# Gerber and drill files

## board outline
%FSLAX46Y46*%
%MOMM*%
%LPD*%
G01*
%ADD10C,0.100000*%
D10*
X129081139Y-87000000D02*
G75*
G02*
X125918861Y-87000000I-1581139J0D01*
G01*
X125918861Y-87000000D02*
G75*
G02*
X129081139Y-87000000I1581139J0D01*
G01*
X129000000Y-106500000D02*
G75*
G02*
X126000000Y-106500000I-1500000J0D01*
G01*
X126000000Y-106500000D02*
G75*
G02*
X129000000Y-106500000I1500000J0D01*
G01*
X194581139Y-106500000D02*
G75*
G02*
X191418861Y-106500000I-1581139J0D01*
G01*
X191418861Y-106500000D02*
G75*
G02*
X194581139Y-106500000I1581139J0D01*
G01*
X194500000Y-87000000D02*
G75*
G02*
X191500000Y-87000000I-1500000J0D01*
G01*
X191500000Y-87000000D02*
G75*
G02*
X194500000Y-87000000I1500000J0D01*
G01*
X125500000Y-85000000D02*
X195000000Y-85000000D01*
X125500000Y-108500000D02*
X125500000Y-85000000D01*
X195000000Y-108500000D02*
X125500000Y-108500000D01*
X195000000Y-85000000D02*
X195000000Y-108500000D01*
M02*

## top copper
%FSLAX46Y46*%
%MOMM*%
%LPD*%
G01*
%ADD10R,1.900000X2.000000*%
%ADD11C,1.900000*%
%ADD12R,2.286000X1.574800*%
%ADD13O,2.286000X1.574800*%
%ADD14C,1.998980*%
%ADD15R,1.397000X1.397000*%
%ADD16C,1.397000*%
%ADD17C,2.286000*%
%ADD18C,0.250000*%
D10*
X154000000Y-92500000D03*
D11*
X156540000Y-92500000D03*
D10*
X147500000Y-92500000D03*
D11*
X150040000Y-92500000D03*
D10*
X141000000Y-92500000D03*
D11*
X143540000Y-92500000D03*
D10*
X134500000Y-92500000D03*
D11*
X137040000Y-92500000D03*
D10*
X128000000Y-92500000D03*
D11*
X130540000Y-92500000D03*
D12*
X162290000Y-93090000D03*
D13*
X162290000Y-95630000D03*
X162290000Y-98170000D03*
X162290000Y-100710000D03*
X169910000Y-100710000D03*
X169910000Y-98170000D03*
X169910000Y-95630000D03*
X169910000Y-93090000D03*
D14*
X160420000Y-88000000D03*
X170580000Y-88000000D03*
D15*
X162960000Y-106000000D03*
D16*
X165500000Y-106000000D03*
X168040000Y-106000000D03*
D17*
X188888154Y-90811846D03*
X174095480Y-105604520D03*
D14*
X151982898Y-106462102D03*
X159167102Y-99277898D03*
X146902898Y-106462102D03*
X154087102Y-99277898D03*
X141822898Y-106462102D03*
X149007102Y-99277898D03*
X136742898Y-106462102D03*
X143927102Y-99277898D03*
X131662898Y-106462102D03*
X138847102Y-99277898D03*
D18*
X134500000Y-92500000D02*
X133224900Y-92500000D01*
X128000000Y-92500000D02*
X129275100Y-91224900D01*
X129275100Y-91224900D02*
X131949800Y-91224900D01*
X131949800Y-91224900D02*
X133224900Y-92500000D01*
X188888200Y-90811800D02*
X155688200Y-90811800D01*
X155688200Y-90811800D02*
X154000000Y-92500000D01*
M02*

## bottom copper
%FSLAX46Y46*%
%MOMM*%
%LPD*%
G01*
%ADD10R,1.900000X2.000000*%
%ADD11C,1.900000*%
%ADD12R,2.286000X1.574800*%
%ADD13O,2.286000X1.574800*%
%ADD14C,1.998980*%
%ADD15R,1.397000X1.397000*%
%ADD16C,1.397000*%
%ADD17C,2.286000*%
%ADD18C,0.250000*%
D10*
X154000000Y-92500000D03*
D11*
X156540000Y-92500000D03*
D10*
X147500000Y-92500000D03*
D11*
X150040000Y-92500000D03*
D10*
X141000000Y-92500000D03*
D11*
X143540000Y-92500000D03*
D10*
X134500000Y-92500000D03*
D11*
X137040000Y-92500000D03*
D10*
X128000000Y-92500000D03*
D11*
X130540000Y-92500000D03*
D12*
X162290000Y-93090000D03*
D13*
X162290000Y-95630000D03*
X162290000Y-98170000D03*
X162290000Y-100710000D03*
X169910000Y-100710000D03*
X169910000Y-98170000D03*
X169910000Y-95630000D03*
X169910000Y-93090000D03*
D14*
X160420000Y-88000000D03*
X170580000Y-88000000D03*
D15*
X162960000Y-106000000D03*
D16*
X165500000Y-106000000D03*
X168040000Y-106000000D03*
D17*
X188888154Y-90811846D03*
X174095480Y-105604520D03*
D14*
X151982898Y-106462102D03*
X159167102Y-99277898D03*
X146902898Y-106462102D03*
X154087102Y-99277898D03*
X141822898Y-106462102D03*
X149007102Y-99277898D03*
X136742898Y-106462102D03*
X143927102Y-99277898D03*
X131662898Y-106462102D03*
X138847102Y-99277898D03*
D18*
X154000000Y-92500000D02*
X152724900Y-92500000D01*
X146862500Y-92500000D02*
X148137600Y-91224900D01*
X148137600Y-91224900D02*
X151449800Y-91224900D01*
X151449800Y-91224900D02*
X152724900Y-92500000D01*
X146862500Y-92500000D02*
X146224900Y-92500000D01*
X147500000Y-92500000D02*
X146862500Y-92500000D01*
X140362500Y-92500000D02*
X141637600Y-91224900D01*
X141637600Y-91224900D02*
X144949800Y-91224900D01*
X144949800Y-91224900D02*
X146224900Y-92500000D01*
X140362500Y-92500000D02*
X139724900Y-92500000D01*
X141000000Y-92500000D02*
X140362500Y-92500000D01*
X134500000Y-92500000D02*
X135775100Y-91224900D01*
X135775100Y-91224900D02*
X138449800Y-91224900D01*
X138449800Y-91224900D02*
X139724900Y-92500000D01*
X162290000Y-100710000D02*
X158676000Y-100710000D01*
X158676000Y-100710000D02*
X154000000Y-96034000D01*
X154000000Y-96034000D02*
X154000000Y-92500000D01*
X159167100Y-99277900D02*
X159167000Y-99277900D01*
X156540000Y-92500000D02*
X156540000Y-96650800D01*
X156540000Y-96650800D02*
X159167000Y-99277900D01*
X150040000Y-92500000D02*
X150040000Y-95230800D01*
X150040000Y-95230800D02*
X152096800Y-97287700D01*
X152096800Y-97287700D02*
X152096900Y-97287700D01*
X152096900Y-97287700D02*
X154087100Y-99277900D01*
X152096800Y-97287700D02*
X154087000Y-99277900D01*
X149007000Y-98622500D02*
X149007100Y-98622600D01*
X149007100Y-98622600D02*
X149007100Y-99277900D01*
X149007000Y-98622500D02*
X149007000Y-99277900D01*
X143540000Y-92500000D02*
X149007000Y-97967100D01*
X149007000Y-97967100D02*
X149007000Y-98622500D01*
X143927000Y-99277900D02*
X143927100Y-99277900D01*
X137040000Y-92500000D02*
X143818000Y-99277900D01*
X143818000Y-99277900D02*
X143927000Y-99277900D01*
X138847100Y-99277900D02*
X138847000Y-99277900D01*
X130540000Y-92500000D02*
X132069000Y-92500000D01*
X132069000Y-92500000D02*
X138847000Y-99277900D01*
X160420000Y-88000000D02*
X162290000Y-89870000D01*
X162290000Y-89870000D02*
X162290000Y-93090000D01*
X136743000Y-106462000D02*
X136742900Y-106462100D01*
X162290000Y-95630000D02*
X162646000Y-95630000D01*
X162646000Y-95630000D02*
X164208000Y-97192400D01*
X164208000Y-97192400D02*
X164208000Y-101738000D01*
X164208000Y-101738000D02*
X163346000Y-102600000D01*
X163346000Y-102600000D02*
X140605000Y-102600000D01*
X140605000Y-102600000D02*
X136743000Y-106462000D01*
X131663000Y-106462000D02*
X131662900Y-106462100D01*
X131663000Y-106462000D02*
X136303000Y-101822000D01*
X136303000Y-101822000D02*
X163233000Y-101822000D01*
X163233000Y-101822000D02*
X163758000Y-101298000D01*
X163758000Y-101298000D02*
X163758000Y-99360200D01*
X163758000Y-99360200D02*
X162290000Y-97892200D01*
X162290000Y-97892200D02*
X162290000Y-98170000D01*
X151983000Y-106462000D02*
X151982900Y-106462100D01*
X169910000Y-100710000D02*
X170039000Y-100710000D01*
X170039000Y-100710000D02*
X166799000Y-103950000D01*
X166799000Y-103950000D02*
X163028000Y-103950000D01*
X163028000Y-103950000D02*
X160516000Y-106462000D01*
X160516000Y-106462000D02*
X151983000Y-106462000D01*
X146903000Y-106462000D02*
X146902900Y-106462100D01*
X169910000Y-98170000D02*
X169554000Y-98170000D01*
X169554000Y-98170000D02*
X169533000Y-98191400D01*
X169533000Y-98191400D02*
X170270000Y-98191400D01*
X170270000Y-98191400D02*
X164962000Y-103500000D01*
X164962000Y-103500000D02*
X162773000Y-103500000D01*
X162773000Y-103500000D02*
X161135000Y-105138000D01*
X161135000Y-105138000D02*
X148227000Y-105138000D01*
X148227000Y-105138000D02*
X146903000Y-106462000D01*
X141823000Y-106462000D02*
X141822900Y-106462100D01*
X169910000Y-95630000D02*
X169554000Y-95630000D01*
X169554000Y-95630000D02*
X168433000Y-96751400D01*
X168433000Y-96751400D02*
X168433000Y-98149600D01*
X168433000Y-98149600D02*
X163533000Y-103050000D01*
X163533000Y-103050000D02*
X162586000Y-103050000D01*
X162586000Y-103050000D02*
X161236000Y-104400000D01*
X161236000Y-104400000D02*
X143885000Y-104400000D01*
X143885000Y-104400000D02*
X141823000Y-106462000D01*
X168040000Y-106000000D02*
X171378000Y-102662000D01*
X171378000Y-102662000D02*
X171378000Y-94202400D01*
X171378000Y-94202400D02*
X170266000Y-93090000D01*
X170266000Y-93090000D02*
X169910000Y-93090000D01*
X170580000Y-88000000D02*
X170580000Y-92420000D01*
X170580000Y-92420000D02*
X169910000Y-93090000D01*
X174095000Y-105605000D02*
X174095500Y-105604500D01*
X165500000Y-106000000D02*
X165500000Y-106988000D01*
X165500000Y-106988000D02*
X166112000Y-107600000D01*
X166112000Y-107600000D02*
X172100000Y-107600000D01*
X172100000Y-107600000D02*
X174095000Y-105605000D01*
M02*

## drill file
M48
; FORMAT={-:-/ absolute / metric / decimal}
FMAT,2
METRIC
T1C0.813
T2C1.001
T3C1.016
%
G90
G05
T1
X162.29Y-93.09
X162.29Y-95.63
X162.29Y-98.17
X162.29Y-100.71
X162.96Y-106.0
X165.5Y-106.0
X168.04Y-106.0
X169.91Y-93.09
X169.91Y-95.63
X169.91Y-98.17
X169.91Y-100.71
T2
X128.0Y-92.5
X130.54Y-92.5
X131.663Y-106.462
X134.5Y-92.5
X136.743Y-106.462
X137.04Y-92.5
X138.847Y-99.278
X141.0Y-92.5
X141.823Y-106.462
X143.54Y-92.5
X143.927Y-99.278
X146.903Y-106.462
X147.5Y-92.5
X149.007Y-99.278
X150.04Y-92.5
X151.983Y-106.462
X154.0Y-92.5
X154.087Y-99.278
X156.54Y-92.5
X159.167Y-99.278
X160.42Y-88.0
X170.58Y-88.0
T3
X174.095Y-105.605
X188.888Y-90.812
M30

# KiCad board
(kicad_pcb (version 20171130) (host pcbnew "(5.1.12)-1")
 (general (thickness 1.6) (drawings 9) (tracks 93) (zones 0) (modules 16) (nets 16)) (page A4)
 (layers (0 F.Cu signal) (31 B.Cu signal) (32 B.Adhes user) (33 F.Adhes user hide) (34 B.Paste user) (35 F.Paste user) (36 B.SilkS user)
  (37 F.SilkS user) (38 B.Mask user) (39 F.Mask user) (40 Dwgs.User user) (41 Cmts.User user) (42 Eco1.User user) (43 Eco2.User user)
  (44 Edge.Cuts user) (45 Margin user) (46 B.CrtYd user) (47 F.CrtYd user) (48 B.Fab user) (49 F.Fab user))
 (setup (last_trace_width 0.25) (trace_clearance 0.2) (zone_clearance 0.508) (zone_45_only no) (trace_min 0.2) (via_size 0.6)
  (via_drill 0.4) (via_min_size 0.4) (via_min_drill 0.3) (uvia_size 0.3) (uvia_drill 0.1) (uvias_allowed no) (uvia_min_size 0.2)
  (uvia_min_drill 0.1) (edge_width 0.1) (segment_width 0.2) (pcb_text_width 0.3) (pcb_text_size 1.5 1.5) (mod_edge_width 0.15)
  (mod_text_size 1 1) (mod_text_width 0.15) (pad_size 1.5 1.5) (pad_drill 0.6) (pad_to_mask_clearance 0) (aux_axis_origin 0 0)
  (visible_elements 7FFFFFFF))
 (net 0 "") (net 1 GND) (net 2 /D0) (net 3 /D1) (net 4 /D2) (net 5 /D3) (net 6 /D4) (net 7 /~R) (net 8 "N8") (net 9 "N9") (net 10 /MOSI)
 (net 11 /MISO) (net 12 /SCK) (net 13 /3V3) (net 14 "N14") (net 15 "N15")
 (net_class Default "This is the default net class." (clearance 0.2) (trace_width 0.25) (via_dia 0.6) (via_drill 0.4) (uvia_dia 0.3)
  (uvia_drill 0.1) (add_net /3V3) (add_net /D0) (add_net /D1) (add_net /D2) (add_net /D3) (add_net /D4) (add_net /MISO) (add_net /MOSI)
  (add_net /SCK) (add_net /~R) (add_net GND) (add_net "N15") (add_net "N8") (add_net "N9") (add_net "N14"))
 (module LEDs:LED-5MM (layer F.Cu) (at 154 92.5)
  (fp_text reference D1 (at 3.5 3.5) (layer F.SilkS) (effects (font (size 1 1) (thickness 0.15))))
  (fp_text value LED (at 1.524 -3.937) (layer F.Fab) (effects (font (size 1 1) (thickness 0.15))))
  (pad 1 thru_hole rect (at 0 0 90) (size 2 1.9) (drill 1.00076) (layers *.Cu *.Mask F.SilkS) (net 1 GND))
  (pad 2 thru_hole circle (at 2.54 0) (size 1.9 1.9) (drill 1.00076) (layers *.Cu *.Mask F.SilkS) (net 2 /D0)))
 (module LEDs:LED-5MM (layer F.Cu) (at 147.5 92.5)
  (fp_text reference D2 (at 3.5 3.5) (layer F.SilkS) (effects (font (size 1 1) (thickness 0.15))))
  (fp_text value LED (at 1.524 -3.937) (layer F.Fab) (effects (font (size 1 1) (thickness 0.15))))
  (pad 1 thru_hole rect (at 0 0 90) (size 2 1.9) (drill 1.00076) (layers *.Cu *.Mask F.SilkS) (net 1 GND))
  (pad 2 thru_hole circle (at 2.54 0) (size 1.9 1.9) (drill 1.00076) (layers *.Cu *.Mask F.SilkS) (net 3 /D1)))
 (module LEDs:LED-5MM (layer F.Cu) (at 141 92.5)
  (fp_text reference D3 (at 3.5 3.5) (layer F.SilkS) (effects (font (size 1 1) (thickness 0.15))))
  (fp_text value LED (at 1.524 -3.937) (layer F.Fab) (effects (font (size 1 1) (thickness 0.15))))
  (pad 1 thru_hole rect (at 0 0 90) (size 2 1.9) (drill 1.00076) (layers *.Cu *.Mask F.SilkS) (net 1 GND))
  (pad 2 thru_hole circle (at 2.54 0) (size 1.9 1.9) (drill 1.00076) (layers *.Cu *.Mask F.SilkS) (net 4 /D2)))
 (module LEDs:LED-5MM (layer F.Cu) (at 134.5 92.5)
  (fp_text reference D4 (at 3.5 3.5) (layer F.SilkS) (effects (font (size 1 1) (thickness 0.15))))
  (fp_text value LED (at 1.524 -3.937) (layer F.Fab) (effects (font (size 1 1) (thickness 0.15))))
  (pad 1 thru_hole rect (at 0 0 90) (size 2 1.9) (drill 1.00076) (layers *.Cu *.Mask F.SilkS) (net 1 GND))
  (pad 2 thru_hole circle (at 2.54 0) (size 1.9 1.9) (drill 1.00076) (layers *.Cu *.Mask F.SilkS) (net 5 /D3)))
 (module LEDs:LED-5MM (layer F.Cu) (at 128 92.5)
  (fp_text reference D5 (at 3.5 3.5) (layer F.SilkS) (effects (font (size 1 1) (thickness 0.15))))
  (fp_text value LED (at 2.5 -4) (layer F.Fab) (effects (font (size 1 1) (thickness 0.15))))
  (pad 1 thru_hole rect (at 0 0 90) (size 2 1.9) (drill 1.00076) (layers *.Cu *.Mask F.SilkS) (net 1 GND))
  (pad 2 thru_hole circle (at 2.54 0) (size 1.9 1.9) (drill 1.00076) (layers *.Cu *.Mask F.SilkS) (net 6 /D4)))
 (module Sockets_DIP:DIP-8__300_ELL (layer F.Cu) (at 166.1 96.9 270)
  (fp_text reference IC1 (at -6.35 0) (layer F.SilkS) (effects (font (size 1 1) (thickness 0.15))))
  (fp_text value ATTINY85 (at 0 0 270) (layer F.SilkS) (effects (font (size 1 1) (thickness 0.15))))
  (pad 1 thru_hole rect (at -3.81 3.81 270) (size 1.5748 2.286) (drill 0.8128) (layers *.Cu *.Mask F.SilkS) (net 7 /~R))
  (pad 2 thru_hole oval (at -1.27 3.81 270) (size 1.5748 2.286) (drill 0.8128) (layers *.Cu *.Mask F.SilkS) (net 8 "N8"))
  (pad 3 thru_hole oval (at 1.27 3.81 270) (size 1.5748 2.286) (drill 0.8128) (layers *.Cu *.Mask F.SilkS) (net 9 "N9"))
  (pad 4 thru_hole oval (at 3.81 3.81 270) (size 1.5748 2.286) (drill 0.8128) (layers *.Cu *.Mask F.SilkS) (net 1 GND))
  (pad 5 thru_hole oval (at 3.81 -3.81 270) (size 1.5748 2.286) (drill 0.8128) (layers *.Cu *.Mask F.SilkS) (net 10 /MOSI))
  (pad 6 thru_hole oval (at 1.27 -3.81 270) (size 1.5748 2.286) (drill 0.8128) (layers *.Cu *.Mask F.SilkS) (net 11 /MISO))
  (pad 7 thru_hole oval (at -1.27 -3.81 270) (size 1.5748 2.286) (drill 0.8128) (layers *.Cu *.Mask F.SilkS) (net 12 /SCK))
  (pad 8 thru_hole oval (at -3.81 -3.81 270) (size 1.5748 2.286) (drill 0.8128) (layers *.Cu *.Mask F.SilkS) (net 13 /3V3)))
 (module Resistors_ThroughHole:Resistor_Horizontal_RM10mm (layer F.Cu) (at 165.5 88)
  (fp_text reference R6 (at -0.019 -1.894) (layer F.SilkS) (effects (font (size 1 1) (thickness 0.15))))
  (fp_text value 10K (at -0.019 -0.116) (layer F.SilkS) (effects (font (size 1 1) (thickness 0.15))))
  (pad 1 thru_hole circle (at -5.08 0) (size 1.99898 1.99898) (drill 1.00076) (layers *.Cu *.SilkS *.Mask) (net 7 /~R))
  (pad 2 thru_hole circle (at 5.08 0) (size 1.99898 1.99898) (drill 1.00076) (layers *.Cu *.SilkS *.Mask) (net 13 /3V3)))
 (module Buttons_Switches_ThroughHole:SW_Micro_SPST (layer F.Cu) (at 165.5 106)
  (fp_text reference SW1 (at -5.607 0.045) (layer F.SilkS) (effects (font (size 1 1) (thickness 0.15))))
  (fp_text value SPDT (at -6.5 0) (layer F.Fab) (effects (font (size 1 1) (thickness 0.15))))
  (pad 1 thru_hole rect (at -2.54 0) (size 1.397 1.397) (drill 0.8128) (layers *.Cu *.Mask F.SilkS) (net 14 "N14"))
  (pad 2 thru_hole circle (at 0 0) (size 1.397 1.397) (drill 0.8128) (layers *.Cu *.Mask F.SilkS) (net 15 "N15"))
  (pad 3 thru_hole circle (at 2.54 0) (size 1.397 1.397) (drill 0.8128) (layers *.Cu *.Mask F.SilkS) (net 13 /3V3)))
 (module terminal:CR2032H (layer F.Cu) (at 183.5 96.2 225)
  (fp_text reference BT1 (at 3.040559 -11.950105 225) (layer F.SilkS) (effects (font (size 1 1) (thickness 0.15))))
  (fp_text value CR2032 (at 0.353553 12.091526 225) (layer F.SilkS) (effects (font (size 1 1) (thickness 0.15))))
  (pad 2 thru_hole circle (at -7.62 0 225) (size 2.286 2.286) (drill 1.016) (layers *.Cu *.Mask F.SilkS) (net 1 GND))
  (pad 1 thru_hole circle (at 13.3 0 225) (size 2.286 2.286) (drill 1.016) (layers *.Cu *.Mask F.SilkS) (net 15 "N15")))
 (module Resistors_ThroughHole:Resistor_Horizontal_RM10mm (layer F.Cu) (at 155.575 102.87 45)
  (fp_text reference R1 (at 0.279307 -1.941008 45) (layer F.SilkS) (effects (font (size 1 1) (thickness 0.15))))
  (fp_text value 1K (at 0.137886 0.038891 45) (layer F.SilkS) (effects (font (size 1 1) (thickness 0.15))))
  (pad 1 thru_hole circle (at -5.08 0 45) (size 1.99898 1.99898) (drill 1.00076) (layers *.Cu *.SilkS *.Mask) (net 10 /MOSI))
  (pad 2 thru_hole circle (at 5.08 0 45) (size 1.99898 1.99898) (drill 1.00076) (layers *.Cu *.SilkS *.Mask) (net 2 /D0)))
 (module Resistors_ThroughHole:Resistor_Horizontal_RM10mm (layer F.Cu) (at 150.495 102.87 45)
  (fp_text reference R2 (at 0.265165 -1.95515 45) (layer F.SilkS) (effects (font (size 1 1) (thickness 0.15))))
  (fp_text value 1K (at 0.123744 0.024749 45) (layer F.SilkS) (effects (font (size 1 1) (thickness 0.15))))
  (pad 1 thru_hole circle (at -5.08 0 45) (size 1.99898 1.99898) (drill 1.00076) (layers *.Cu *.SilkS *.Mask) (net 11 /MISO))
  (pad 2 thru_hole circle (at 5.08 0 45) (size 1.99898 1.99898) (drill 1.00076) (layers *.Cu *.SilkS *.Mask) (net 3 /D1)))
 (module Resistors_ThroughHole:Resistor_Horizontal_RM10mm (layer F.Cu) (at 145.415 102.87 45)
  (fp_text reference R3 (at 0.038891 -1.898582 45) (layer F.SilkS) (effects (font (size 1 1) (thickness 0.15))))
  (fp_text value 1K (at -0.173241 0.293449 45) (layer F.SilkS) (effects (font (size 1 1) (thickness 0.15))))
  (pad 1 thru_hole circle (at -5.08 0 45) (size 1.99898 1.99898) (drill 1.00076) (layers *.Cu *.SilkS *.Mask) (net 12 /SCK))
  (pad 2 thru_hole circle (at 5.08 0 45) (size 1.99898 1.99898) (drill 1.00076) (layers *.Cu *.SilkS *.Mask) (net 4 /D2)))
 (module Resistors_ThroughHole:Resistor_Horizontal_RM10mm (layer F.Cu) (at 140.335 102.87 45)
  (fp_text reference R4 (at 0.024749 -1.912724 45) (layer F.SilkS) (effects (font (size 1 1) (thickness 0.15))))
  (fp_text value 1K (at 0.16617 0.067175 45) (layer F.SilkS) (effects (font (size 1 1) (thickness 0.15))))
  (pad 1 thru_hole circle (at -5.08 0 45) (size 1.99898 1.99898) (drill 1.00076) (layers *.Cu *.SilkS *.Mask) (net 8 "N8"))
  (pad 2 thru_hole circle (at 5.08 0 45) (size 1.99898 1.99898) (drill 1.00076) (layers *.Cu *.SilkS *.Mask) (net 5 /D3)))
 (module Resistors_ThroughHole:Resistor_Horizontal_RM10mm (layer F.Cu) (at 135.255 102.87 45)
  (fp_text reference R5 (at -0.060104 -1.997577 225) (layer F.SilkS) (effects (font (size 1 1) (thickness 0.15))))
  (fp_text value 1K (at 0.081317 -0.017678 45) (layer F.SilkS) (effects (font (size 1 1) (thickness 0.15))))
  (pad 1 thru_hole circle (at -5.08 0 45) (size 1.99898 1.99898) (drill 1.00076) (layers *.Cu *.SilkS *.Mask) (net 9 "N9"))
  (pad 2 thru_hole circle (at 5.08 0 45) (size 1.99898 1.99898) (drill 1.00076) (layers *.Cu *.SilkS *.Mask) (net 6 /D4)))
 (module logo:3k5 (layer F.Cu) (at 140.589 87.503)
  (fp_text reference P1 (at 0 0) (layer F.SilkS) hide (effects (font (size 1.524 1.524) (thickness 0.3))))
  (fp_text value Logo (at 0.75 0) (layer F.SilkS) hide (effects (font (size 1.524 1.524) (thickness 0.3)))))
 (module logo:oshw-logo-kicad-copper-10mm (layer F.Cu) (at 129.413 99.187)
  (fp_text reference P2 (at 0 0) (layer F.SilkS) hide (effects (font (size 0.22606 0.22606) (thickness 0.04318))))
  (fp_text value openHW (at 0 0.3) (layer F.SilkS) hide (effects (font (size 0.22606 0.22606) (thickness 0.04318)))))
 (gr_circle (center 127.5 87) (end 129 87.5) (layer Edge.Cuts) (width 0.1))
 (gr_circle (center 127.5 106.5) (end 129 106.5) (layer Edge.Cuts) (width 0.1))
 (gr_circle (center 193 106.5) (end 194.5 107) (layer Edge.Cuts) (width 0.1))
 (gr_circle (center 193 87) (end 194.5 87) (layer Edge.Cuts) (width 0.1))
 (gr_line (start 125.5 85) (end 195 85) (angle 90) (layer Edge.Cuts) (width 0.1))
 (gr_line (start 125.5 108.5) (end 125.5 85) (angle 90) (layer Edge.Cuts) (width 0.1))
 (gr_line (start 195 108.5) (end 125.5 108.5) (angle 90) (layer Edge.Cuts) (width 0.1))
 (gr_line (start 195 85) (end 195 108.5) (angle 90) (layer Edge.Cuts) (width 0.1))
 (segment (start 154 92.5) (end 152.7249 92.5) (width 0.25) (layer B.Cu) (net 1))
 (segment (start 146.8625 92.5) (end 148.1376 91.2249) (width 0.25) (layer B.Cu) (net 1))
 (segment (start 148.1376 91.2249) (end 151.4498 91.2249) (width 0.25) (layer B.Cu) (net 1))
 (segment (start 151.4498 91.2249) (end 152.7249 92.5) (width 0.25) (layer B.Cu) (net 1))
 (segment (start 146.8625 92.5) (end 146.2249 92.5) (width 0.25) (layer B.Cu) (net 1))
 (segment (start 147.5 92.5) (end 146.8625 92.5) (width 0.25) (layer B.Cu) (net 1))
 (segment (start 140.3625 92.5) (end 141.6376 91.2249) (width 0.25) (layer B.Cu) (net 1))
 (segment (start 141.6376 91.2249) (end 144.9498 91.2249) (width 0.25) (layer B.Cu) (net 1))
 (segment (start 144.9498 91.2249) (end 146.2249 92.5) (width 0.25) (layer B.Cu) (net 1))
 (segment (start 140.3625 92.5) (end 139.7249 92.5) (width 0.25) (layer B.Cu) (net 1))
 (segment (start 141 92.5) (end 140.3625 92.5) (width 0.25) (layer B.Cu) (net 1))
 (segment (start 134.5 92.5) (end 135.7751 91.2249) (width 0.25) (layer B.Cu) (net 1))
 (segment (start 135.7751 91.2249) (end 138.4498 91.2249) (width 0.25) (layer B.Cu) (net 1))
 (segment (start 138.4498 91.2249) (end 139.7249 92.5) (width 0.25) (layer B.Cu) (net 1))
 (segment (start 134.5 92.5) (end 133.2249 92.5) (width 0.25) (layer F.Cu) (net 1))
 (segment (start 128 92.5) (end 129.2751 91.2249) (width 0.25) (layer F.Cu) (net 1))
 (segment (start 129.2751 91.2249) (end 131.9498 91.2249) (width 0.25) (layer F.Cu) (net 1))
 (segment (start 131.9498 91.2249) (end 133.2249 92.5) (width 0.25) (layer F.Cu) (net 1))
 (segment (start 162.29 100.71) (end 158.676 100.71) (width 0.25) (layer B.Cu) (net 1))
 (segment (start 158.676 100.71) (end 154 96.034) (width 0.25) (layer B.Cu) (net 1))
 (segment (start 154 96.034) (end 154 92.5) (width 0.25) (layer B.Cu) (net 1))
 (segment (start 188.8882 90.8118) (end 155.6882 90.8118) (width 0.25) (layer F.Cu) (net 1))
 (segment (start 155.6882 90.8118) (end 154 92.5) (width 0.25) (layer F.Cu) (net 1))
 (segment (start 159.1671 99.2779) (end 159.167 99.2779) (width 0.25) (layer B.Cu) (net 2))
 (segment (start 156.54 92.5) (end 156.54 96.6508) (width 0.25) (layer B.Cu) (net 2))
 (segment (start 156.54 96.6508) (end 159.167 99.2779) (width 0.25) (layer B.Cu) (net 2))
 (segment (start 150.04 92.5) (end 150.04 95.2308) (width 0.25) (layer B.Cu) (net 3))
 (segment (start 150.04 95.2308) (end 152.0968 97.2877) (width 0.25) (layer B.Cu) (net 3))
 (segment (start 152.0968 97.2877) (end 152.0969 97.2877) (width 0.25) (layer B.Cu) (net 3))
 (segment (start 152.0969 97.2877) (end 154.0871 99.2779) (width 0.25) (layer B.Cu) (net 3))
 (segment (start 152.0968 97.2877) (end 154.087 99.2779) (width 0.25) (layer B.Cu) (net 3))
 (segment (start 149.007 98.6225) (end 149.0071 98.6226) (width 0.25) (layer B.Cu) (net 4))
 (segment (start 149.0071 98.6226) (end 149.0071 99.2779) (width 0.25) (layer B.Cu) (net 4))
 (segment (start 149.007 98.6225) (end 149.007 99.2779) (width 0.25) (layer B.Cu) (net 4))
 (segment (start 143.54 92.5) (end 149.007 97.9671) (width 0.25) (layer B.Cu) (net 4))
 (segment (start 149.007 97.9671) (end 149.007 98.6225) (width 0.25) (layer B.Cu) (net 4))
 (segment (start 143.927 99.2779) (end 143.9271 99.2779) (width 0.25) (layer B.Cu) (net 5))
 (segment (start 137.04 92.5) (end 143.818 99.2779) (width 0.25) (layer B.Cu) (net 5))
 (segment (start 143.818 99.2779) (end 143.927 99.2779) (width 0.25) (layer B.Cu) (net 5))
 (segment (start 138.8471 99.2779) (end 138.847 99.2779) (width 0.25) (layer B.Cu) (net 6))
 (segment (start 130.54 92.5) (end 132.069 92.5) (width 0.25) (layer B.Cu) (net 6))
 (segment (start 132.069 92.5) (end 138.847 99.2779) (width 0.25) (layer B.Cu) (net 6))
 (segment (start 160.42 88) (end 162.29 89.87) (width 0.25) (layer B.Cu) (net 7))
 (segment (start 162.29 89.87) (end 162.29 93.09) (width 0.25) (layer B.Cu) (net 7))
 (segment (start 136.743 106.462) (end 136.7429 106.4621) (width 0.25) (layer B.Cu) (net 8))
 (segment (start 162.29 95.63) (end 162.646 95.63) (width 0.25) (layer B.Cu) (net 8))
 (segment (start 162.646 95.63) (end 164.208 97.1924) (width 0.25) (layer B.Cu) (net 8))
 (segment (start 164.208 97.1924) (end 164.208 101.738) (width 0.25) (layer B.Cu) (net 8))
 (segment (start 164.208 101.738) (end 163.346 102.6) (width 0.25) (layer B.Cu) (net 8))
 (segment (start 163.346 102.6) (end 140.605 102.6) (width 0.25) (layer B.Cu) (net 8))
 (segment (start 140.605 102.6) (end 136.743 106.462) (width 0.25) (layer B.Cu) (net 8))
 (segment (start 131.663 106.462) (end 131.6629 106.4621) (width 0.25) (layer B.Cu) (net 9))
 (segment (start 131.663 106.462) (end 136.303 101.822) (width 0.25) (layer B.Cu) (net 9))
 (segment (start 136.303 101.822) (end 163.233 101.822) (width 0.25) (layer B.Cu) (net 9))
 (segment (start 163.233 101.822) (end 163.758 101.298) (width 0.25) (layer B.Cu) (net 9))
 (segment (start 163.758 101.298) (end 163.758 99.3602) (width 0.25) (layer B.Cu) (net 9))
 (segment (start 163.758 99.3602) (end 162.29 97.8922) (width 0.25) (layer B.Cu) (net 9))
 (segment (start 162.29 97.8922) (end 162.29 98.17) (width 0.25) (layer B.Cu) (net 9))
 (segment (start 151.983 106.462) (end 151.9829 106.4621) (width 0.25) (layer B.Cu) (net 10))
 (segment (start 169.91 100.71) (end 170.039 100.71) (width 0.25) (layer B.Cu) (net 10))
 (segment (start 170.039 100.71) (end 166.799 103.95) (width 0.25) (layer B.Cu) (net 10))
 (segment (start 166.799 103.95) (end 163.028 103.95) (width 0.25) (layer B.Cu) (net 10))
 (segment (start 163.028 103.95) (end 160.516 106.462) (width 0.25) (layer B.Cu) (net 10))
 (segment (start 160.516 106.462) (end 151.983 106.462) (width 0.25) (layer B.Cu) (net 10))
 (segment (start 146.903 106.462) (end 146.9029 106.4621) (width 0.25) (layer B.Cu) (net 11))
 (segment (start 169.91 98.17) (end 169.554 98.17) (width 0.25) (layer B.Cu) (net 11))
 (segment (start 169.554 98.17) (end 169.533 98.1914) (width 0.25) (layer B.Cu) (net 11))
 (segment (start 169.533 98.1914) (end 170.27 98.1914) (width 0.25) (layer B.Cu) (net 11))
 (segment (start 170.27 98.1914) (end 164.962 103.5) (width 0.25) (layer B.Cu) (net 11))
 (segment (start 164.962 103.5) (end 162.773 103.5) (width 0.25) (layer B.Cu) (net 11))
 (segment (start 162.773 103.5) (end 161.135 105.138) (width 0.25) (layer B.Cu) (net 11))
 (segment (start 161.135 105.138) (end 148.227 105.138) (width 0.25) (layer B.Cu) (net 11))
 (segment (start 148.227 105.138) (end 146.903 106.462) (width 0.25) (layer B.Cu) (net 11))
 (segment (start 141.823 106.462) (end 141.8229 106.4621) (width 0.25) (layer B.Cu) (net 12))
 (segment (start 169.91 95.63) (end 169.554 95.63) (width 0.25) (layer B.Cu) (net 12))
 (segment (start 169.554 95.63) (end 168.433 96.7514) (width 0.25) (layer B.Cu) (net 12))
 (segment (start 168.433 96.7514) (end 168.433 98.1496) (width 0.25) (layer B.Cu) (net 12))
 (segment (start 168.433 98.1496) (end 163.533 103.05) (width 0.25) (layer B.Cu) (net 12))
 (segment (start 163.533 103.05) (end 162.586 103.05) (width 0.25) (layer B.Cu) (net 12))
 (segment (start 162.586 103.05) (end 161.236 104.4) (width 0.25) (layer B.Cu) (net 12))
 (segment (start 161.236 104.4) (end 143.885 104.4) (width 0.25) (layer B.Cu) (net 12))
 (segment (start 143.885 104.4) (end 141.823 106.462) (width 0.25) (layer B.Cu) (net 12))
 (segment (start 168.04 106) (end 171.378 102.662) (width 0.25) (layer B.Cu) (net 13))
 (segment (start 171.378 102.662) (end 171.378 94.2024) (width 0.25) (layer B.Cu) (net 13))
 (segment (start 171.378 94.2024) (end 170.266 93.09) (width 0.25) (layer B.Cu) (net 13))
 (segment (start 170.266 93.09) (end 169.91 93.09) (width 0.25) (layer B.Cu) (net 13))
 (segment (start 170.58 88) (end 170.58 92.42) (width 0.25) (layer B.Cu) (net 13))
 (segment (start 170.58 92.42) (end 169.91 93.09) (width 0.25) (layer B.Cu) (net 13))
 (segment (start 174.095 105.605) (end 174.0955 105.6045) (width 0.25) (layer B.Cu) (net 15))
 (segment (start 165.5 106) (end 165.5 106.988) (width 0.25) (layer B.Cu) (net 15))
 (segment (start 165.5 106.988) (end 166.112 107.6) (width 0.25) (layer B.Cu) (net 15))
 (segment (start 166.112 107.6) (end 172.1 107.6) (width 0.25) (layer B.Cu) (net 15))
 (segment (start 172.1 107.6) (end 174.095 105.605) (width 0.25) (layer B.Cu) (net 15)))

